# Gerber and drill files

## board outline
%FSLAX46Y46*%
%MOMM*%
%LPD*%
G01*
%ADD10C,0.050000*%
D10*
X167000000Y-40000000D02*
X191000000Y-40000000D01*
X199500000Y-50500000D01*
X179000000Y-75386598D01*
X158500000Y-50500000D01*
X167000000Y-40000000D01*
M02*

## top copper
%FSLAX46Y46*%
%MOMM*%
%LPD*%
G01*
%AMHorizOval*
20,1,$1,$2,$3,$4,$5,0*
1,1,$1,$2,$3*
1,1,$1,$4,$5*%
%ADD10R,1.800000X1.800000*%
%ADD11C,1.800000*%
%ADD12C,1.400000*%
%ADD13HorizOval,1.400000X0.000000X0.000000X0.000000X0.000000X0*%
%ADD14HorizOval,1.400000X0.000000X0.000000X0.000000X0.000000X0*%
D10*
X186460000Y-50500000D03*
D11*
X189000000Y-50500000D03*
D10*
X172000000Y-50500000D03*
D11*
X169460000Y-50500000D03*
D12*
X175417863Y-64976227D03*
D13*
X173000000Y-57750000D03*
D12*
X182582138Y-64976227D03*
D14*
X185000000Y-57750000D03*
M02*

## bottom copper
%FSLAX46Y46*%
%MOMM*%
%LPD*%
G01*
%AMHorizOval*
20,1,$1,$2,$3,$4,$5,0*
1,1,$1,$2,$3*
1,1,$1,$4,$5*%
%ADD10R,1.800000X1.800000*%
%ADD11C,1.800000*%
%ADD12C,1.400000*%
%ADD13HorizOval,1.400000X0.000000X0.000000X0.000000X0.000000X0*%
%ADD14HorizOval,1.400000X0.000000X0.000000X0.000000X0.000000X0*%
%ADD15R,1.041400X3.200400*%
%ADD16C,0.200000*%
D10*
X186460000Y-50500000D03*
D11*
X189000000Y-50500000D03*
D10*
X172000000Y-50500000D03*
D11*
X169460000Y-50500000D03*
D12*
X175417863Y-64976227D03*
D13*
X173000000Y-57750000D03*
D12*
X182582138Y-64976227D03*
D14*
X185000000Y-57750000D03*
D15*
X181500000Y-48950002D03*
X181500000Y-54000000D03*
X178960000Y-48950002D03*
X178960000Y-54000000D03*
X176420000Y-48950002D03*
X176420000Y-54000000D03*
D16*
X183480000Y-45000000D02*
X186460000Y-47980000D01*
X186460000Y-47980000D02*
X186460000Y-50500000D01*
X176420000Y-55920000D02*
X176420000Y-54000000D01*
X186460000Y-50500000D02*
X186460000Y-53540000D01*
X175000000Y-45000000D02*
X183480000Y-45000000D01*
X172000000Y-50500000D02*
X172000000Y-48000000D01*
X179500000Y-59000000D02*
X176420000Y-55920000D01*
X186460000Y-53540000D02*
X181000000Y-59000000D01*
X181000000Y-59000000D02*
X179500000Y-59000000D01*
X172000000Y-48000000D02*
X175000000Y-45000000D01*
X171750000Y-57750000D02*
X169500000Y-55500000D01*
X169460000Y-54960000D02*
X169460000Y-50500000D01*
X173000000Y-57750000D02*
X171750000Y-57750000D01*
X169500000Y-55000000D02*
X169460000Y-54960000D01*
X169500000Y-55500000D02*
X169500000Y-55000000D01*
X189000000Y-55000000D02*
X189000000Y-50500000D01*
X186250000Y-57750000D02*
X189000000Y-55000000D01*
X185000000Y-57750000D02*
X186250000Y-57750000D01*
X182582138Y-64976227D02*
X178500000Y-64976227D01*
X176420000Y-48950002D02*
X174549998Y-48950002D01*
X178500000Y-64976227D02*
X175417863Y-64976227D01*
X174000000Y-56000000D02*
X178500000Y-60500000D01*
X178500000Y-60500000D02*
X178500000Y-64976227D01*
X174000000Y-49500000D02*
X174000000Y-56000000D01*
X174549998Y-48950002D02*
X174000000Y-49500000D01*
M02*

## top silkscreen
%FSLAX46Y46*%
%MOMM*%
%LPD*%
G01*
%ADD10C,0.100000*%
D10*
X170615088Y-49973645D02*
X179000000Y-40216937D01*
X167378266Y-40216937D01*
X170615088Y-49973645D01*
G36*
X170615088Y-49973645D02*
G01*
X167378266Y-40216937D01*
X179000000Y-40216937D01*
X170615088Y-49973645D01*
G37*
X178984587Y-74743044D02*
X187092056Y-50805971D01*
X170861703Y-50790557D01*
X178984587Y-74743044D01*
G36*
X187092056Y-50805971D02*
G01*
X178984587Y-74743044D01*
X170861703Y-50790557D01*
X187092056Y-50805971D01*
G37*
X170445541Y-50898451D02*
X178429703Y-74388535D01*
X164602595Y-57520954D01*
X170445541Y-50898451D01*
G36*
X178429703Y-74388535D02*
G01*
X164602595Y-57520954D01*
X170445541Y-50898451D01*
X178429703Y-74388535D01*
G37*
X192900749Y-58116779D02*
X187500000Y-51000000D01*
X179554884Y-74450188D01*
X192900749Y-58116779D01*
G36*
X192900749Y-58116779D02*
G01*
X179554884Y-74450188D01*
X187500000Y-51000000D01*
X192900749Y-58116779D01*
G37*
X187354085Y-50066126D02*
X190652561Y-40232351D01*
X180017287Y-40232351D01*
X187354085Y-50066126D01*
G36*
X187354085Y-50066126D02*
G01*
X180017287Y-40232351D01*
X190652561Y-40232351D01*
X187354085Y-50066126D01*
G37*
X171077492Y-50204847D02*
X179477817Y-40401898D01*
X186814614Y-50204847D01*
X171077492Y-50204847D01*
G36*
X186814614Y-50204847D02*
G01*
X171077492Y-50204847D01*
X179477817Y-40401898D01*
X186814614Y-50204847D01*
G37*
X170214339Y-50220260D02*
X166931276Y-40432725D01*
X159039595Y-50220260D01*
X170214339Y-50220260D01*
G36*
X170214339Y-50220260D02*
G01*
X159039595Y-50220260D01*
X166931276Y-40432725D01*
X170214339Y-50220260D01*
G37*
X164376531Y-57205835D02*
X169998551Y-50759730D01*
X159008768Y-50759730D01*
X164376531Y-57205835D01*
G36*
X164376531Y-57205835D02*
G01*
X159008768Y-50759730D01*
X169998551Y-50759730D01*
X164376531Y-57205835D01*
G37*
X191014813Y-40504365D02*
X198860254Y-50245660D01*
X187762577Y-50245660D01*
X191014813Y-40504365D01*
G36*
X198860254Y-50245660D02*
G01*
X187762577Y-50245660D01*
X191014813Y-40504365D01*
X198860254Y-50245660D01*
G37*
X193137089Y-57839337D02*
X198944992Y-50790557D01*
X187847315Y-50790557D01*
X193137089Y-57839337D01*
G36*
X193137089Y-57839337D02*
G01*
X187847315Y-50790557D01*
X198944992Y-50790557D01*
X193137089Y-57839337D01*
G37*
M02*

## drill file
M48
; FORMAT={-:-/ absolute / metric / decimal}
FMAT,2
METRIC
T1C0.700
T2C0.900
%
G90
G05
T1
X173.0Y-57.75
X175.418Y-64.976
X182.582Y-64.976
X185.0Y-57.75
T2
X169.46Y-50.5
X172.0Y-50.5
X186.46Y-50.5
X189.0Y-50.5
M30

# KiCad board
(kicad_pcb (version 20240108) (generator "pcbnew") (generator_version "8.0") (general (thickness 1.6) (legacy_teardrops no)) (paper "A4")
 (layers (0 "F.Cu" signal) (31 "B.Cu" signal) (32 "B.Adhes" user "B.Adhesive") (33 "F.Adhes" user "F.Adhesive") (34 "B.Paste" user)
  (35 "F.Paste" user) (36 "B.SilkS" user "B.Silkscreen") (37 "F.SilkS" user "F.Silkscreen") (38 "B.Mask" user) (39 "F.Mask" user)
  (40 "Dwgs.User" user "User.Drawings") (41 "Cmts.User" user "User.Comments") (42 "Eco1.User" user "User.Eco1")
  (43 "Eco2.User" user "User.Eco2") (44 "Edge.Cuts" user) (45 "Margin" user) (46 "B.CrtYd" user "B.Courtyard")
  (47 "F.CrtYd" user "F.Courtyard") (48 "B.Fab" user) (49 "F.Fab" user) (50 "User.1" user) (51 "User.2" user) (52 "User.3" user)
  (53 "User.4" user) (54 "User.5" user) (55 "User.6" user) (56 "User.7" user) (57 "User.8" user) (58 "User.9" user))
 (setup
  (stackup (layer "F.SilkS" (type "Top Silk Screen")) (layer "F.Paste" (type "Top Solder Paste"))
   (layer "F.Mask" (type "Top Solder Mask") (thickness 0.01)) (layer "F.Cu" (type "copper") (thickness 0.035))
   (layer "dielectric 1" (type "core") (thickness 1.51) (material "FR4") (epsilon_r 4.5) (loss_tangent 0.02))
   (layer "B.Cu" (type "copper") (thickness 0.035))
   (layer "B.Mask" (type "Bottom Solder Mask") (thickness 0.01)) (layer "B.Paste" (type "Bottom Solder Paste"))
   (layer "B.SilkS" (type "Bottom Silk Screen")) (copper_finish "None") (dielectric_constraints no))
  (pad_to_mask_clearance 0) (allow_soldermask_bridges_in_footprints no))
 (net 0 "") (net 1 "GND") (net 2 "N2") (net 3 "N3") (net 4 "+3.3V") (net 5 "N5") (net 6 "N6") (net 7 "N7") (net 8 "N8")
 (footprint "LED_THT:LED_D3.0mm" (layer "F.Cu") (at 186.46 50.5)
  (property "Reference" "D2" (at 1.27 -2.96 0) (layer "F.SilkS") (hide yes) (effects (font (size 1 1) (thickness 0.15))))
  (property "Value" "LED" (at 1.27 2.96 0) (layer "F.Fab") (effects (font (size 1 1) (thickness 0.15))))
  (pad "1" thru_hole rect (at 0 0) (size 1.8 1.8) (drill 0.9) (layers "*.Cu" "*.Mask") (remove_unused_layers no) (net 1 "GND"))
  (pad "2" thru_hole circle (at 2.54 0) (size 1.8 1.8) (drill 0.9) (layers "*.Cu" "*.Mask") (remove_unused_layers no) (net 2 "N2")))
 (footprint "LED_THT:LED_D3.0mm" (layer "F.Cu") (at 172 50.5 180)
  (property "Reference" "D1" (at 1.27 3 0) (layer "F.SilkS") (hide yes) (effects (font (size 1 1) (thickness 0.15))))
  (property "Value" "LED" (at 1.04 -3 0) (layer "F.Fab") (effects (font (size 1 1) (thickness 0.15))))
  (pad "1" thru_hole rect (at 0 0 180) (size 1.8 1.8) (drill 0.9) (layers "*.Cu" "*.Mask") (remove_unused_layers no) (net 1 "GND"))
  (pad "2" thru_hole circle (at 2.54 0 180) (size 1.8 1.8) (drill 0.9) (layers "*.Cu" "*.Mask") (remove_unused_layers no) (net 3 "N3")))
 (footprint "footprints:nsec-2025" (layer "B.Cu") (at 185.6 46.65 180)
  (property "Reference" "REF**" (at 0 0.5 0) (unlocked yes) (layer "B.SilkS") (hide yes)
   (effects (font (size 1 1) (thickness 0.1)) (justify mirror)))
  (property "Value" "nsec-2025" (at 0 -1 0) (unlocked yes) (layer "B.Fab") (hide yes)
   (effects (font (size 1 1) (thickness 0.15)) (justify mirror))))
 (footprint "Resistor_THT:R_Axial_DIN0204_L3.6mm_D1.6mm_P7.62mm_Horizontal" (layer "B.Cu") (at 175.417863 64.976227 108.5)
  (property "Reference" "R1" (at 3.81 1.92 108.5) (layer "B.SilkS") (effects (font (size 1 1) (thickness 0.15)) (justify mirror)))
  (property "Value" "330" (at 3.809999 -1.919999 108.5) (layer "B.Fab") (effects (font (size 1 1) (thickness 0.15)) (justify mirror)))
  (pad "1" thru_hole circle (at 0 0 108.5) (size 1.4 1.4) (drill 0.7) (layers "*.Cu" "*.Mask") (remove_unused_layers no) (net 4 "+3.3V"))
  (pad "2" thru_hole oval (at 7.620001 -0.000001 108.5) (size 1.4 1.4) (drill 0.7) (layers "*.Cu" "*.Mask") (remove_unused_layers no)
   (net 3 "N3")))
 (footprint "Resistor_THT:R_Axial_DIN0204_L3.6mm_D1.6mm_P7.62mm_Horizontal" (layer "B.Cu") (at 182.582138 64.976227 71.5)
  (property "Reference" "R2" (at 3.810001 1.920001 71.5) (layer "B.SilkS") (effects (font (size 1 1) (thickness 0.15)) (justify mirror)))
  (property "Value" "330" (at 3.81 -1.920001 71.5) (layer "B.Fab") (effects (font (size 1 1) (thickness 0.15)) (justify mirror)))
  (pad "1" thru_hole circle (at 0 0 72.5) (size 1.4 1.4) (drill 0.7) (layers "*.Cu" "*.Mask") (remove_unused_layers no) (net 4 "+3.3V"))
  (pad "2" thru_hole oval (at 7.620001 0 71.5) (size 1.4 1.4) (drill 0.7) (layers "*.Cu" "*.Mask") (remove_unused_layers no) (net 2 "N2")))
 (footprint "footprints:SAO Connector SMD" (layer "B.Cu") (at 178.96 51.475001 180)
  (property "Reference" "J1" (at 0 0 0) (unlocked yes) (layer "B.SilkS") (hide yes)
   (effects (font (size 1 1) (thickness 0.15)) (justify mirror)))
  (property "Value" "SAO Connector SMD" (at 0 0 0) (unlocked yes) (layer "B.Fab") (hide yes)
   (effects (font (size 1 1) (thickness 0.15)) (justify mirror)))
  (pad "1" smd rect (at -2.54 2.524999 180) (size 1.0414 3.2004) (layers "B.Cu" "B.Paste" "B.Mask") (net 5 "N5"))
  (pad "2" smd rect (at -2.54 -2.524999 180) (size 1.0414 3.2004) (layers "B.Cu" "B.Paste" "B.Mask") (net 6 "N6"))
  (pad "3" smd rect (at 0 2.524999 180) (size 1.0414 3.2004) (layers "B.Cu" "B.Paste" "B.Mask") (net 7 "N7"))
  (pad "4" smd rect (at 0 -2.524999 180) (size 1.0414 3.2004) (layers "B.Cu" "B.Paste" "B.Mask") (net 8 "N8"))
  (pad "5" smd rect (at 2.54 2.524999 180) (size 1.0414 3.2004) (layers "B.Cu" "B.Paste" "B.Mask") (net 4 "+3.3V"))
  (pad "6" smd rect (at 2.54 -2.524999 180) (size 1.0414 3.2004) (layers "B.Cu" "B.Paste" "B.Mask") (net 1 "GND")))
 (gr_poly
  (pts (xy 170.615088 49.973645) (xy 179 40.216937) (xy 167.378266 40.216937)) (stroke (width 0.1) (type solid)) (fill solid)
  (layer "F.SilkS"))
 (gr_poly
  (pts (xy 178.984587 74.743044) (xy 187.092056 50.805971) (xy 170.861703 50.790557)) (stroke (width 0.1) (type solid)) (fill solid)
  (layer "F.SilkS"))
 (gr_poly
  (pts (xy 170.445541 50.898451) (xy 178.429703 74.388535) (xy 164.602595 57.520954)) (stroke (width 0.1) (type solid)) (fill solid)
  (layer "F.SilkS"))
 (gr_poly
  (pts (xy 192.900749 58.116779) (xy 187.5 51) (xy 179.554884 74.450188)) (stroke (width 0.1) (type solid)) (fill solid) (layer "F.SilkS"))
 (gr_poly
  (pts (xy 187.354085 50.066126) (xy 190.652561 40.232351) (xy 180.017287 40.232351)) (stroke (width 0.1) (type solid)) (fill solid)
  (layer "F.SilkS"))
 (gr_poly
  (pts (xy 171.077492 50.204847) (xy 179.477817 40.401898) (xy 186.814614 50.204847)) (stroke (width 0.1) (type solid)) (fill solid)
  (layer "F.SilkS"))
 (gr_poly
  (pts (xy 170.214339 50.22026) (xy 166.931276 40.432725) (xy 159.039595 50.22026)) (stroke (width 0.1) (type solid)) (fill solid)
  (layer "F.SilkS"))
 (gr_poly
  (pts (xy 164.376531 57.205835) (xy 169.998551 50.75973) (xy 159.008768 50.75973)) (stroke (width 0.1) (type solid)) (fill solid)
  (layer "F.SilkS"))
 (gr_poly
  (pts (xy 191.014813 40.504365) (xy 198.860254 50.24566) (xy 187.762577 50.24566)) (stroke (width 0.1) (type solid)) (fill solid)
  (layer "F.SilkS"))
 (gr_poly
  (pts (xy 193.137089 57.839337) (xy 198.944992 50.790557) (xy 187.847315 50.790557)) (stroke (width 0.1) (type solid)) (fill solid)
  (layer "F.SilkS"))
 (gr_poly
  (pts (xy 167 40) (xy 191 40) (xy 199.5 50.5) (xy 179 75.386598) (xy 158.5 50.5)) (stroke (width 0.05) (type solid)) (fill none)
  (layer "Edge.Cuts"))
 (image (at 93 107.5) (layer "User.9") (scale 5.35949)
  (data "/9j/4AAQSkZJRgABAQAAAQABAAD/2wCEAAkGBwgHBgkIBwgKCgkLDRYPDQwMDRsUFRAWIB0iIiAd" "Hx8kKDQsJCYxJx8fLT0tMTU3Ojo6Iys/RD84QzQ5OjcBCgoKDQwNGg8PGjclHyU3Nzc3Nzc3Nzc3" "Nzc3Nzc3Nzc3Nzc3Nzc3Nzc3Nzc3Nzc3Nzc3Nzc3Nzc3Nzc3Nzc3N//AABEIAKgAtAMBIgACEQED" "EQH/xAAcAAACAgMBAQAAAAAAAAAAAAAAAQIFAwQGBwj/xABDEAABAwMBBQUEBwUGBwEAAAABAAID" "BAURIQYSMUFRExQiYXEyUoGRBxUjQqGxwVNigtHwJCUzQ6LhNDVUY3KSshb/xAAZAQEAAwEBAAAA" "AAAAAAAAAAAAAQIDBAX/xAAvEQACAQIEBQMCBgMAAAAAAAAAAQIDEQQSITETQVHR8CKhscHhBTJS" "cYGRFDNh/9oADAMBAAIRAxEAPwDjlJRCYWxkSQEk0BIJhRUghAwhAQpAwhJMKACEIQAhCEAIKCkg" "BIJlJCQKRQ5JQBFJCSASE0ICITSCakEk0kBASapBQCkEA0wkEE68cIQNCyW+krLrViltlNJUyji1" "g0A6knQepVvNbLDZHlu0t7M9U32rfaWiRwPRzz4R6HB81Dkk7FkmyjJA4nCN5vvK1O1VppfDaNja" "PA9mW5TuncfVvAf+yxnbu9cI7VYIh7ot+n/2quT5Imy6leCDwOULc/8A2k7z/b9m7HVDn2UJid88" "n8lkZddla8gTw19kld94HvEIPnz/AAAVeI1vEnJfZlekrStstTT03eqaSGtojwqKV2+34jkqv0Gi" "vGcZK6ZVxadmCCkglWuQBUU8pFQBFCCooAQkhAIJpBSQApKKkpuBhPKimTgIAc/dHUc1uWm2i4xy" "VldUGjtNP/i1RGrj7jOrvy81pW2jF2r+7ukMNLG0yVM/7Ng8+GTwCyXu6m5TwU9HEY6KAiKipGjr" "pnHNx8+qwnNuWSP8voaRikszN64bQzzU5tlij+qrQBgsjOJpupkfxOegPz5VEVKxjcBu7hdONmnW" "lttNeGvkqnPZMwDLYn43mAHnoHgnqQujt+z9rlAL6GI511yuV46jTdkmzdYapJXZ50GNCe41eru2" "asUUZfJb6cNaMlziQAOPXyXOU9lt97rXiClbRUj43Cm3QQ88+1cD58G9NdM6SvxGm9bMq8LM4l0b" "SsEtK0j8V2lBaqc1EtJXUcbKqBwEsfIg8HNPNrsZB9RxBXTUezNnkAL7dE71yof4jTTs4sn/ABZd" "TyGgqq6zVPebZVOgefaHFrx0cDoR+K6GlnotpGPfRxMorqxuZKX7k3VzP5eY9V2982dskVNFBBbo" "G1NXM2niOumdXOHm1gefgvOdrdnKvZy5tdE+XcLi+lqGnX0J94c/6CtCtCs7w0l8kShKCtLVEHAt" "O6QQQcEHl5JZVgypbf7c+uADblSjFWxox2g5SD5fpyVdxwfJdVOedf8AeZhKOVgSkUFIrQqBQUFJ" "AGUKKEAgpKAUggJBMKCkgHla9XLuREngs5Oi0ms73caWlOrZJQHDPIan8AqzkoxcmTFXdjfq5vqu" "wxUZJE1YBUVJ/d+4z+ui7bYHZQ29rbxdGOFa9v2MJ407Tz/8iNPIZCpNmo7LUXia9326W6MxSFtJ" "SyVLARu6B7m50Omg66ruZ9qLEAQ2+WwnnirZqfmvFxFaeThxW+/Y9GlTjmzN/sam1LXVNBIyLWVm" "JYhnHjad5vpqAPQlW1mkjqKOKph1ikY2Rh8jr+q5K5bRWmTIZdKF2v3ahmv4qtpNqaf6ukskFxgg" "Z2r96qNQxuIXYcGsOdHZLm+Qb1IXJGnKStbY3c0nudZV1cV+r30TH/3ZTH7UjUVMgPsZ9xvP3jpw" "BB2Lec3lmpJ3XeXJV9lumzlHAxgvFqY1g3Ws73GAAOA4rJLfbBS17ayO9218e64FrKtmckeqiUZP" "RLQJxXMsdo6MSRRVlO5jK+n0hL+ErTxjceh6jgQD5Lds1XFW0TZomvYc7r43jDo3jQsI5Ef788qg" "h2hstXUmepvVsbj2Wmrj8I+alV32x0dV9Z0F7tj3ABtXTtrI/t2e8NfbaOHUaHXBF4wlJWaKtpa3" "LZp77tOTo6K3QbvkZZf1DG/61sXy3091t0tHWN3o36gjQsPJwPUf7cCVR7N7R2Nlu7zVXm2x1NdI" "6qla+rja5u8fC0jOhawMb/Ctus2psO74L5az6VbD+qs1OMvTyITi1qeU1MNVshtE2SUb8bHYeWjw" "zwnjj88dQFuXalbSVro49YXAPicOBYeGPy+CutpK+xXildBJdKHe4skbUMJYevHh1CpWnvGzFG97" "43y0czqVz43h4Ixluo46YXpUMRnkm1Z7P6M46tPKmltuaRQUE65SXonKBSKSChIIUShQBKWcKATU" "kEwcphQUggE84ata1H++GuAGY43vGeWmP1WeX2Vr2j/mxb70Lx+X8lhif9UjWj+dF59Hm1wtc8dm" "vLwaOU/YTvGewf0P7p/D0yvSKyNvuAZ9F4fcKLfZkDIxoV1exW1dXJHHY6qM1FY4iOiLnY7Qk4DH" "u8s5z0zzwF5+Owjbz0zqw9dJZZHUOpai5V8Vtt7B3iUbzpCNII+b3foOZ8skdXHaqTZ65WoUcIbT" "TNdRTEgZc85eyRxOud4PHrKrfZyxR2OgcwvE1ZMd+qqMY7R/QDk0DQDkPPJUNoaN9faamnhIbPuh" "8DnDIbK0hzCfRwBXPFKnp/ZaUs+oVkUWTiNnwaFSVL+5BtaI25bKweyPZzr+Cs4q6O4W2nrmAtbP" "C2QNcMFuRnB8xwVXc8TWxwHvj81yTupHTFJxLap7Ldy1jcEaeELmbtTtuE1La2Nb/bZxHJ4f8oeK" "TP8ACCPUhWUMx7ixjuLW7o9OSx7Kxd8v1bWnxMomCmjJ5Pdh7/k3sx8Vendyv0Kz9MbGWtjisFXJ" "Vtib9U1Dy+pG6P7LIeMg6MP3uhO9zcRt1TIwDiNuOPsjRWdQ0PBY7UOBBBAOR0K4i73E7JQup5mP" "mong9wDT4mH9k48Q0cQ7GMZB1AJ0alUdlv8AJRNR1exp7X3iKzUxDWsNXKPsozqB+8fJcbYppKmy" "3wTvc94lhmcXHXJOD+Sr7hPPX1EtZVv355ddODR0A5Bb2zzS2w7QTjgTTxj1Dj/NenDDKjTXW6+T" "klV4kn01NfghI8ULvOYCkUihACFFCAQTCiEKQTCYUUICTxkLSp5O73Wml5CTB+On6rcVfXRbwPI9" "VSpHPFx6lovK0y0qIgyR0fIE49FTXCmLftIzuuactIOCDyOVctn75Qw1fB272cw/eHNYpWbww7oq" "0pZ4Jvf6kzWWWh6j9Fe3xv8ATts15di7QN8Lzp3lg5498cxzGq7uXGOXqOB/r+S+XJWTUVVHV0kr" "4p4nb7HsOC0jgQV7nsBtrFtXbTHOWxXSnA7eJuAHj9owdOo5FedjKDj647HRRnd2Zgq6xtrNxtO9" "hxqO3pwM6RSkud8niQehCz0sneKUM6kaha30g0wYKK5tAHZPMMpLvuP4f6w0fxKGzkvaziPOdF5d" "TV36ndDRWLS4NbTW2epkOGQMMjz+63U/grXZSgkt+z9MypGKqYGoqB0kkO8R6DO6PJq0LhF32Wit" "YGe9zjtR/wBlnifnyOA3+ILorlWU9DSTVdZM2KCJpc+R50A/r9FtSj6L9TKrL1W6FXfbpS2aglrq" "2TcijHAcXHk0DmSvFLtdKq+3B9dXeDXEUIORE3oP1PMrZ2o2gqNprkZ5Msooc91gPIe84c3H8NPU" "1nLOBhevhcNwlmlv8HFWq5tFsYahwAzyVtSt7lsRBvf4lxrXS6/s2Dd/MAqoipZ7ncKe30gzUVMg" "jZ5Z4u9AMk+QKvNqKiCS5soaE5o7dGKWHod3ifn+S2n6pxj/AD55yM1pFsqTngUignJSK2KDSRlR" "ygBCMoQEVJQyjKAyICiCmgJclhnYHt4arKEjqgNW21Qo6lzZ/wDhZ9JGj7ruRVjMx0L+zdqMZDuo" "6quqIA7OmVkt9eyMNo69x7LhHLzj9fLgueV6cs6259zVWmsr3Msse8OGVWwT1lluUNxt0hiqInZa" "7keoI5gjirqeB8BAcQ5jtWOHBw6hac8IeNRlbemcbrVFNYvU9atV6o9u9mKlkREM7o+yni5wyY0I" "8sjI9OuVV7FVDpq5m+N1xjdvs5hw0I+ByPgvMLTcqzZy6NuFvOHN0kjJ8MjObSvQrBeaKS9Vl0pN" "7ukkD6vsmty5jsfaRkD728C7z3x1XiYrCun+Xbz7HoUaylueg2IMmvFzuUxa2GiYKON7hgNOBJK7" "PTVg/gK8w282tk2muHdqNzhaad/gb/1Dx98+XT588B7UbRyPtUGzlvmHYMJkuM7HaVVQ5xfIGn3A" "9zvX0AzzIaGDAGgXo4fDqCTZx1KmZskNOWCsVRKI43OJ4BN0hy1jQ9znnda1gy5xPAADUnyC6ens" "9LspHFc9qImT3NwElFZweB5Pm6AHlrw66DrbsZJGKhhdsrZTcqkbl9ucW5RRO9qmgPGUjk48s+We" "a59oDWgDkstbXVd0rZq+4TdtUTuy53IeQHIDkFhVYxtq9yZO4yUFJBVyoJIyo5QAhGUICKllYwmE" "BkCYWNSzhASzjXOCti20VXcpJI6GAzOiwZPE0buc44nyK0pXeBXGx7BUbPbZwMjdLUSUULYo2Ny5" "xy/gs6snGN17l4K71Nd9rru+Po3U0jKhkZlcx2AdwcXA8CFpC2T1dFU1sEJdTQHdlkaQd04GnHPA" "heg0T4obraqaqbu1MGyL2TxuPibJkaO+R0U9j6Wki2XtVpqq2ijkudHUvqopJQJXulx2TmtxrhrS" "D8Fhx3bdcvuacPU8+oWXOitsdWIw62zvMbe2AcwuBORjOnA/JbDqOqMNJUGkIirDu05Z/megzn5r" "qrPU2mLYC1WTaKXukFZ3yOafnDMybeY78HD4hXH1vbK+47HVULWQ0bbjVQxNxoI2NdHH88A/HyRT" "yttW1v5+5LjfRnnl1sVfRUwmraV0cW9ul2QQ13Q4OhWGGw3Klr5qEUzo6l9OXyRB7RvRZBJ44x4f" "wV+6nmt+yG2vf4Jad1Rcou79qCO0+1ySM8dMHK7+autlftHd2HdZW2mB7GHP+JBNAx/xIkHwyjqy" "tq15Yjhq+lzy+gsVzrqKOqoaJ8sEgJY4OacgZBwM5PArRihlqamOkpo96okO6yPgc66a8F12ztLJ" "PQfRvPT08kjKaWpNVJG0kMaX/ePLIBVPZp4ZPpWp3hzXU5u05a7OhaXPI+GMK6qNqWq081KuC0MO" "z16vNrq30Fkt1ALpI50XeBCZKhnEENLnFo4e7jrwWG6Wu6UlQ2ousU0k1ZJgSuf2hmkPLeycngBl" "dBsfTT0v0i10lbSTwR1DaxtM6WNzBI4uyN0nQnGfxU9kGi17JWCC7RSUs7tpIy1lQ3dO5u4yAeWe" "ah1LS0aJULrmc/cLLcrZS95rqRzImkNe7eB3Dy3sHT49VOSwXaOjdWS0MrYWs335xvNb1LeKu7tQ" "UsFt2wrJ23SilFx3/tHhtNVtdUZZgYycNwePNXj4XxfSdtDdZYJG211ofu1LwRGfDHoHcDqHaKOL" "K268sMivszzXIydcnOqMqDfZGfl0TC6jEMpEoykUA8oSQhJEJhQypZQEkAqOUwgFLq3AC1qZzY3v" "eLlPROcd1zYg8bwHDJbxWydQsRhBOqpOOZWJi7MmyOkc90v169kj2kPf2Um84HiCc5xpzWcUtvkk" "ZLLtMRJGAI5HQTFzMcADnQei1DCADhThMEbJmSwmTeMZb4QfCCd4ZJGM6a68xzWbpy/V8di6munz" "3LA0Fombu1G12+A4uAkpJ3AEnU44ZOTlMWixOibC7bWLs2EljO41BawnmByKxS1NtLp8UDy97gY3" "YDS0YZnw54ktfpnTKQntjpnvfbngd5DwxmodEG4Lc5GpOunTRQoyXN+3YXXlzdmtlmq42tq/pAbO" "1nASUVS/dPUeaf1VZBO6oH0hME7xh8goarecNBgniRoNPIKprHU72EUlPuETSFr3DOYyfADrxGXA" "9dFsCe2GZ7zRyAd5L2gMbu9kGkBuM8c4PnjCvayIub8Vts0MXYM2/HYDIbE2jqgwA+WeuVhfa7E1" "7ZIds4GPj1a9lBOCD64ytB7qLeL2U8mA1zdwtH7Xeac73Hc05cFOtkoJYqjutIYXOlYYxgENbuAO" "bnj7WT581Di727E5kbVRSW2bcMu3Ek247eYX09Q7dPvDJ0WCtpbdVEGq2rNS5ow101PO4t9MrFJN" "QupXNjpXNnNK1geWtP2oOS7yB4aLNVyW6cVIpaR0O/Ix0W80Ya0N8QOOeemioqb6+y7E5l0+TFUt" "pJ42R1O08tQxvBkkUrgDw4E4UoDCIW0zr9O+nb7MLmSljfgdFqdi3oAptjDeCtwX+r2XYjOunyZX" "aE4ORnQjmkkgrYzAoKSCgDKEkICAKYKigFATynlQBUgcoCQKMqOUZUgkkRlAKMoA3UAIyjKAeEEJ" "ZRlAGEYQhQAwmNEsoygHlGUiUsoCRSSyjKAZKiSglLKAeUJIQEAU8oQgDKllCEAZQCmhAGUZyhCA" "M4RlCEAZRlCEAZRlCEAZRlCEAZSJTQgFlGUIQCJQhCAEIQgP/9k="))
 (segment (start 183.48 45) (end 186.46 47.98) (width 0.2) (layer "B.Cu") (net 1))
 (segment (start 186.46 47.98) (end 186.46 50.5) (width 0.2) (layer "B.Cu") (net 1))
 (segment (start 176.42 55.92) (end 176.42 54) (width 0.2) (layer "B.Cu") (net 1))
 (segment (start 186.46 50.5) (end 186.46 53.54) (width 0.2) (layer "B.Cu") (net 1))
 (segment (start 175 45) (end 183.48 45) (width 0.2) (layer "B.Cu") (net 1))
 (segment (start 172 50.5) (end 172 48) (width 0.2) (layer "B.Cu") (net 1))
 (segment (start 179.5 59) (end 176.42 55.92) (width 0.2) (layer "B.Cu") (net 1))
 (segment (start 186.46 53.54) (end 181 59) (width 0.2) (layer "B.Cu") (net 1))
 (segment (start 181 59) (end 179.5 59) (width 0.2) (layer "B.Cu") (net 1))
 (segment (start 172 48) (end 175 45) (width 0.2) (layer "B.Cu") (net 1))
 (segment (start 171.75 57.75) (end 169.5 55.5) (width 0.2) (layer "B.Cu") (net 3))
 (segment (start 169.46 54.96) (end 169.46 50.5) (width 0.2) (layer "B.Cu") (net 3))
 (segment (start 173 57.75) (end 171.75 57.75) (width 0.2) (layer "B.Cu") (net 3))
 (segment (start 169.5 55) (end 169.46 54.96) (width 0.2) (layer "B.Cu") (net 3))
 (segment (start 169.5 55.5) (end 169.5 55) (width 0.2) (layer "B.Cu") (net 3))
 (segment (start 189 55) (end 189 50.5) (width 0.2) (layer "B.Cu") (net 2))
 (segment (start 186.25 57.75) (end 189 55) (width 0.2) (layer "B.Cu") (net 2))
 (segment (start 185 57.75) (end 186.25 57.75) (width 0.2) (layer "B.Cu") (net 2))
 (segment (start 182.582138 64.976227) (end 178.5 64.976227) (width 0.2) (layer "B.Cu") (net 4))
 (segment (start 176.42 48.950002) (end 174.549998 48.950002) (width 0.2) (layer "B.Cu") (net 4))
 (segment (start 178.5 64.976227) (end 175.417863 64.976227) (width 0.2) (layer "B.Cu") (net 4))
 (segment (start 174 56) (end 178.5 60.5) (width 0.2) (layer "B.Cu") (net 4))
 (segment (start 178.5 60.5) (end 178.5 64.976227) (width 0.2) (layer "B.Cu") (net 4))
 (segment (start 174 49.5) (end 174 56) (width 0.2) (layer "B.Cu") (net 4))
 (segment (start 174.549998 48.950002) (end 174 49.5) (width 0.2) (layer "B.Cu") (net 4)))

